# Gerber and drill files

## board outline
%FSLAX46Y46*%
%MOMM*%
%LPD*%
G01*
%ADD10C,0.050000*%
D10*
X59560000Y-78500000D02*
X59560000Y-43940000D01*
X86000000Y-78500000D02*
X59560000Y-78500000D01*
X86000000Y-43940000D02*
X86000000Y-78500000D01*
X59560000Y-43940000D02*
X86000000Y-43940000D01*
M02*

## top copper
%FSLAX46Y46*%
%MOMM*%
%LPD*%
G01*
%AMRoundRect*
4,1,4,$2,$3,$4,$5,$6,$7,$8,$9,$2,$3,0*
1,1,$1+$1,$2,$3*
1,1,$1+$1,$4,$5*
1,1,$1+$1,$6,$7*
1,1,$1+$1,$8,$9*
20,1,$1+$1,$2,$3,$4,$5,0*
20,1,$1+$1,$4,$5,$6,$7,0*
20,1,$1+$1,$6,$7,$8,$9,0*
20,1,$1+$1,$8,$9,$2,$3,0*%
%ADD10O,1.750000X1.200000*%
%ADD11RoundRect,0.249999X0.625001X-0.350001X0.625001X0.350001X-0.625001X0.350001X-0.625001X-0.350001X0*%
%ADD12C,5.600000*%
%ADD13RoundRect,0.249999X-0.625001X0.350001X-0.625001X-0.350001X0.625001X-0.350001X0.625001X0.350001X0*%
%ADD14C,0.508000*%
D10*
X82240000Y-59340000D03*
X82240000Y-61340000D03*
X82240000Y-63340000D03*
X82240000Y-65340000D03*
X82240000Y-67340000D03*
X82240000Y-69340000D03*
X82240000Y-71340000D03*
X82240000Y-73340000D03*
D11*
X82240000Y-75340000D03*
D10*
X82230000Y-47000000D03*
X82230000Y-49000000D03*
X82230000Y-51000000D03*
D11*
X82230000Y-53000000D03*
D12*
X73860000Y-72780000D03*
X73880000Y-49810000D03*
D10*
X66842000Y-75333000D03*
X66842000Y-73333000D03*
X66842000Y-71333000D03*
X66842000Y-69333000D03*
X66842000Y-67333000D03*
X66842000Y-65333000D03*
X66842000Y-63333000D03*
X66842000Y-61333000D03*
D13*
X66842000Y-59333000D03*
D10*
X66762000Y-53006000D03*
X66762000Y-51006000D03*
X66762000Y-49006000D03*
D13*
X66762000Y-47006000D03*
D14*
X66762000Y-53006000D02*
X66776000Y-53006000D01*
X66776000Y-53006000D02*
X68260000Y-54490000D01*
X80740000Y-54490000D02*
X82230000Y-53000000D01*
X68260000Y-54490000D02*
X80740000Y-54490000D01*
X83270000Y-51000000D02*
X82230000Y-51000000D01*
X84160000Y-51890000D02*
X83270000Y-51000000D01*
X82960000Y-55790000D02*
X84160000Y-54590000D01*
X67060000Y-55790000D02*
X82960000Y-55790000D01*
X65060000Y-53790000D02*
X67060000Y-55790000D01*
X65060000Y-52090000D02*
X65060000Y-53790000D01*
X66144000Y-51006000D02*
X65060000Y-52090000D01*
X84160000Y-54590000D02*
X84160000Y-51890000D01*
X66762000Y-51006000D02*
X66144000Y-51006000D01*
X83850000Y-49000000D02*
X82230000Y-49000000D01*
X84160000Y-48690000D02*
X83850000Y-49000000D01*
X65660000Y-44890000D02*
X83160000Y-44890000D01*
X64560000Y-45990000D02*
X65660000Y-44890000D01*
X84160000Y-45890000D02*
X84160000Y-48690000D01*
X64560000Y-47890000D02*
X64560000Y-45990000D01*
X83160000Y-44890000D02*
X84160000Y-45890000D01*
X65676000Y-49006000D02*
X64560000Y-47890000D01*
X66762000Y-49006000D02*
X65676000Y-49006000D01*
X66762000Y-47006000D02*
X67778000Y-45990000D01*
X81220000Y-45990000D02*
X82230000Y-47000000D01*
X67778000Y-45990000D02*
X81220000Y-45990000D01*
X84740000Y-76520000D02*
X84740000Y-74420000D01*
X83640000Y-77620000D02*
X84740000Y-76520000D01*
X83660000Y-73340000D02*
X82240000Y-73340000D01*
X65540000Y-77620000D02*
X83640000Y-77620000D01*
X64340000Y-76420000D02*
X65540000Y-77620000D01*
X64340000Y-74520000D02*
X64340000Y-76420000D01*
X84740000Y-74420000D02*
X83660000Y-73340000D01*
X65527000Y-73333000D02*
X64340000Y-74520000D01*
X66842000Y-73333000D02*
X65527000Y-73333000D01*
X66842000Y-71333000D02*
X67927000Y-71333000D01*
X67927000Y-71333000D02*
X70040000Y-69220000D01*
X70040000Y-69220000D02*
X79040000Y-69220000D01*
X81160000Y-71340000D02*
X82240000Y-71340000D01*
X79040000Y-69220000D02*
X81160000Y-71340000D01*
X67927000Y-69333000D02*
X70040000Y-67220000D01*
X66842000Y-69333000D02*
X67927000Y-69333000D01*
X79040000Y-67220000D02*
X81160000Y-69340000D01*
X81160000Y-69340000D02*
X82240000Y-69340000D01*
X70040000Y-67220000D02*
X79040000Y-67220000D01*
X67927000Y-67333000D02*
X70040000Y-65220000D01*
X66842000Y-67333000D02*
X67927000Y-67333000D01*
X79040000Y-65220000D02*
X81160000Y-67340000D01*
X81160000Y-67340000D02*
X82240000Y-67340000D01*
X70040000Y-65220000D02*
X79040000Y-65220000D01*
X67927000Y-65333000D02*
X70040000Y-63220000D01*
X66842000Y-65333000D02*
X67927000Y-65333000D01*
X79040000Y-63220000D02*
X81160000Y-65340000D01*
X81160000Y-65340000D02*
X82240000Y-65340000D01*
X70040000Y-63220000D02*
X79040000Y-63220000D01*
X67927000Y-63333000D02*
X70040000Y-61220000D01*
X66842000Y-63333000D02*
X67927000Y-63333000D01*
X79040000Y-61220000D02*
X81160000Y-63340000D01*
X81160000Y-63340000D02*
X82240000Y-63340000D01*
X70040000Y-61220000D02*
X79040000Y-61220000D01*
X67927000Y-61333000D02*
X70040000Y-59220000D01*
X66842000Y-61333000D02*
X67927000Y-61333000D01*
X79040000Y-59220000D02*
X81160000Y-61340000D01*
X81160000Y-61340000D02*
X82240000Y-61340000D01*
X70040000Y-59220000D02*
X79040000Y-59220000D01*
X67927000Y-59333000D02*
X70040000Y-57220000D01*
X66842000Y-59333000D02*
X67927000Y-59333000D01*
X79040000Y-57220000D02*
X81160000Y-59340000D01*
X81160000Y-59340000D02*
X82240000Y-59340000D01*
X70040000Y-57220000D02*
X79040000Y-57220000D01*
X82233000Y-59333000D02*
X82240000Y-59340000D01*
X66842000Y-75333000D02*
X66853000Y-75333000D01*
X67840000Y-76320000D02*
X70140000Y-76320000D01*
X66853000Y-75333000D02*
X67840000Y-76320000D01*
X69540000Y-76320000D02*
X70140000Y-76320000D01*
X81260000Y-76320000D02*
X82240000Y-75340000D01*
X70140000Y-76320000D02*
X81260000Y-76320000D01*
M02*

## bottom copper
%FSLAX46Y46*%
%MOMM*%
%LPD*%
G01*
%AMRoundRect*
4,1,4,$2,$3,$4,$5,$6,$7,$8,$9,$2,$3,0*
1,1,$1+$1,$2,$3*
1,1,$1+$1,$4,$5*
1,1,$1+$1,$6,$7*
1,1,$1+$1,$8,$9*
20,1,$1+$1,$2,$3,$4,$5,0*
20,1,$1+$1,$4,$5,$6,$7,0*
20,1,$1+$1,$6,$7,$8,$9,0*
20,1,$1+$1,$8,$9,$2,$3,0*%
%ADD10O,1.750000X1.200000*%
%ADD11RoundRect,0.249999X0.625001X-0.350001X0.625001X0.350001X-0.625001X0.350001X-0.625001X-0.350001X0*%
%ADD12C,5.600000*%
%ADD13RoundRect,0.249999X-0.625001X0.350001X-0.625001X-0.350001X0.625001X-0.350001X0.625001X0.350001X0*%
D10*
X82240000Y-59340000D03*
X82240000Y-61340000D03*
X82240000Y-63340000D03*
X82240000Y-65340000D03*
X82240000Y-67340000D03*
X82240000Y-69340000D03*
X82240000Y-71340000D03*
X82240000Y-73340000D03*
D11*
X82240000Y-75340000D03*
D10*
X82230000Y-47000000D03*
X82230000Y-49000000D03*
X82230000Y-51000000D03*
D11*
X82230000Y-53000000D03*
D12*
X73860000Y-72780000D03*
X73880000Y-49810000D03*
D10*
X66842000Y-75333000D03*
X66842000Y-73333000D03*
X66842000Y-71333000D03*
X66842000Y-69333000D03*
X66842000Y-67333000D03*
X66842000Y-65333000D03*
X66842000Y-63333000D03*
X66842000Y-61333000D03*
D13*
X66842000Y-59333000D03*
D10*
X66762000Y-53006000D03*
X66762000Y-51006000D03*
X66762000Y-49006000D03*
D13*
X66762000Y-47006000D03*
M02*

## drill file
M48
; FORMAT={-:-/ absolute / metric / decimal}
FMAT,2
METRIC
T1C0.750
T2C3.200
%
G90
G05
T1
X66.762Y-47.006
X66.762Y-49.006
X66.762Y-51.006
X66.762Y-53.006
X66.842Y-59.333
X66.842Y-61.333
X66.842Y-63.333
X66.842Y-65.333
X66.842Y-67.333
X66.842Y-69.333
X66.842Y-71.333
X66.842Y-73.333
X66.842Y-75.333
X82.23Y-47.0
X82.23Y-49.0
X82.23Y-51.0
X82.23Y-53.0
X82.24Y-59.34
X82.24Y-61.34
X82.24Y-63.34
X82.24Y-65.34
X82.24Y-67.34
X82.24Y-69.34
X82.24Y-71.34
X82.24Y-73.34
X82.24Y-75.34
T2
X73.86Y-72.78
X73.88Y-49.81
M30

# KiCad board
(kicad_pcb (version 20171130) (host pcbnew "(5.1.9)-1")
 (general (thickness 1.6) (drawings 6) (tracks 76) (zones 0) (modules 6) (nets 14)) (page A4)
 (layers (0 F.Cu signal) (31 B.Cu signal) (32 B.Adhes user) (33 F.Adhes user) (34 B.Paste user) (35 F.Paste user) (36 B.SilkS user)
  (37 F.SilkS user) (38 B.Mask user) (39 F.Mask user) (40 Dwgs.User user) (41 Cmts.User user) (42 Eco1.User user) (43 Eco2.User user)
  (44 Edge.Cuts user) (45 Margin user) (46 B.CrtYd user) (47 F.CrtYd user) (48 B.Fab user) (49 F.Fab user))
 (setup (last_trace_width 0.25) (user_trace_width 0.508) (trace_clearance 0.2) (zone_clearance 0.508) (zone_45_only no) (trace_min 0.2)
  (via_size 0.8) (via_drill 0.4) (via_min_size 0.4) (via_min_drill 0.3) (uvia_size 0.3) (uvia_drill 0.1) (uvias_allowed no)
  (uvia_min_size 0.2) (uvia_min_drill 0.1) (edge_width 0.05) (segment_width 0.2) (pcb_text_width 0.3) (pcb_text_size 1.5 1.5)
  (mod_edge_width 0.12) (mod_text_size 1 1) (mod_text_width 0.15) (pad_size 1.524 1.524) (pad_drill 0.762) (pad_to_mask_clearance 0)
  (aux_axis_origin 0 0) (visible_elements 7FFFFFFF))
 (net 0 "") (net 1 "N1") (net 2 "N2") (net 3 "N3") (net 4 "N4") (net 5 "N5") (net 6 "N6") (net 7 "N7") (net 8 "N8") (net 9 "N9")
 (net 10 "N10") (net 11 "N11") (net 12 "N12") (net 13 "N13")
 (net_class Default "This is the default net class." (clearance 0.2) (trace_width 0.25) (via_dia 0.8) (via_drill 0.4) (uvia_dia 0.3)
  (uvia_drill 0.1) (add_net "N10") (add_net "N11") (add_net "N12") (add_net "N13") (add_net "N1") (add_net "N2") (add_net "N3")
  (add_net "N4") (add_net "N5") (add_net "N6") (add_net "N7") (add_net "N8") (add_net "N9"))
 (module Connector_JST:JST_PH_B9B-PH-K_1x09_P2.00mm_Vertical (layer F.Cu) (at 82.24 75.34 90)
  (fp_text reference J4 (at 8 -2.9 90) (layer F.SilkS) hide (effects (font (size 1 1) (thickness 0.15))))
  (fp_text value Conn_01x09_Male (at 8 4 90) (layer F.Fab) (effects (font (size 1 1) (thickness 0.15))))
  (pad 9 thru_hole oval (at 16 0 90) (size 1.2 1.75) (drill 0.75) (layers *.Cu *.Mask) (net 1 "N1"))
  (pad 8 thru_hole oval (at 14 0 90) (size 1.2 1.75) (drill 0.75) (layers *.Cu *.Mask) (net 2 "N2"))
  (pad 7 thru_hole oval (at 12 0 90) (size 1.2 1.75) (drill 0.75) (layers *.Cu *.Mask) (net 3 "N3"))
  (pad 6 thru_hole oval (at 10 0 90) (size 1.2 1.75) (drill 0.75) (layers *.Cu *.Mask) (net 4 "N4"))
  (pad 5 thru_hole oval (at 8 0 90) (size 1.2 1.75) (drill 0.75) (layers *.Cu *.Mask) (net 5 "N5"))
  (pad 4 thru_hole oval (at 6 0 90) (size 1.2 1.75) (drill 0.75) (layers *.Cu *.Mask) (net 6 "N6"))
  (pad 3 thru_hole oval (at 4 0 90) (size 1.2 1.75) (drill 0.75) (layers *.Cu *.Mask) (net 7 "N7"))
  (pad 2 thru_hole oval (at 2 0 90) (size 1.2 1.75) (drill 0.75) (layers *.Cu *.Mask) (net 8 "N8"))
  (pad 1 thru_hole roundrect (at 0 0 90) (size 1.2 1.75) (drill 0.75) (layers *.Cu *.Mask) (roundrect_rratio 0.2083325) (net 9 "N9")))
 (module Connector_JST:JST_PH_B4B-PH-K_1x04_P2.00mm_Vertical (layer F.Cu) (at 82.23 53 90)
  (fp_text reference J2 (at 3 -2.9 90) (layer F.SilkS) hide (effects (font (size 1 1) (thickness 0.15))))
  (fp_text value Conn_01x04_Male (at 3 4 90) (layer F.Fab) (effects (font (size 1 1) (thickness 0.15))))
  (pad 4 thru_hole oval (at 6 0 90) (size 1.2 1.75) (drill 0.75) (layers *.Cu *.Mask) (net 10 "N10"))
  (pad 3 thru_hole oval (at 4 0 90) (size 1.2 1.75) (drill 0.75) (layers *.Cu *.Mask) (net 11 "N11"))
  (pad 2 thru_hole oval (at 2 0 90) (size 1.2 1.75) (drill 0.75) (layers *.Cu *.Mask) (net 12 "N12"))
  (pad 1 thru_hole roundrect (at 0 0 90) (size 1.2 1.75) (drill 0.75) (layers *.Cu *.Mask) (roundrect_rratio 0.2083325) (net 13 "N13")))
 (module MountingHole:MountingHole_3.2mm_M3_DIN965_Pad (layer F.Cu) (at 73.86 72.78)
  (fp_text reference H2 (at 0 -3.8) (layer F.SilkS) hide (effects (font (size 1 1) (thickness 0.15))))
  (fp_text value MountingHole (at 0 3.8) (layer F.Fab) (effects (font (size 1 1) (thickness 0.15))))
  (pad 1 thru_hole circle (at 0 0) (size 5.6 5.6) (drill 3.2) (layers *.Cu *.Mask)))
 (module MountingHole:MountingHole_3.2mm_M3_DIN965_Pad (layer F.Cu) (at 73.88 49.81)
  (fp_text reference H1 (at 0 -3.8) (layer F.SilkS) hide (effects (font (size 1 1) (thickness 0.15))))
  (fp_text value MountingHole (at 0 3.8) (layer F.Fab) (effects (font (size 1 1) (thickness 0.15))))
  (pad 1 thru_hole circle (at 0 0) (size 5.6 5.6) (drill 3.2) (layers *.Cu *.Mask)))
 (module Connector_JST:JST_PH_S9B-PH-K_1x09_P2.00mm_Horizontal (layer F.Cu) (at 66.842 59.333 270)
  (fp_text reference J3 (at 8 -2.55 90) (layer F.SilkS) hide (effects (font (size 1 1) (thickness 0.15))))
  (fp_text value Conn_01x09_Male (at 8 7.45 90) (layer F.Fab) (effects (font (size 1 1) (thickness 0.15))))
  (pad 9 thru_hole oval (at 16 0 270) (size 1.2 1.75) (drill 0.75) (layers *.Cu *.Mask) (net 9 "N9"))
  (pad 8 thru_hole oval (at 14 0 270) (size 1.2 1.75) (drill 0.75) (layers *.Cu *.Mask) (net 8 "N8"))
  (pad 7 thru_hole oval (at 12 0 270) (size 1.2 1.75) (drill 0.75) (layers *.Cu *.Mask) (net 7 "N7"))
  (pad 6 thru_hole oval (at 10 0 270) (size 1.2 1.75) (drill 0.75) (layers *.Cu *.Mask) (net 6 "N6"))
  (pad 5 thru_hole oval (at 8 0 270) (size 1.2 1.75) (drill 0.75) (layers *.Cu *.Mask) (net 5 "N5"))
  (pad 4 thru_hole oval (at 6 0 270) (size 1.2 1.75) (drill 0.75) (layers *.Cu *.Mask) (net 4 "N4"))
  (pad 3 thru_hole oval (at 4 0 270) (size 1.2 1.75) (drill 0.75) (layers *.Cu *.Mask) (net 3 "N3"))
  (pad 2 thru_hole oval (at 2 0 270) (size 1.2 1.75) (drill 0.75) (layers *.Cu *.Mask) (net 2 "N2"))
  (pad 1 thru_hole roundrect (at 0 0 270) (size 1.2 1.75) (drill 0.75) (layers *.Cu *.Mask) (roundrect_rratio 0.2083325) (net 1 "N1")))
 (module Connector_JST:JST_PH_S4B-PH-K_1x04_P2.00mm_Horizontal (layer F.Cu) (at 66.762 47.006 270)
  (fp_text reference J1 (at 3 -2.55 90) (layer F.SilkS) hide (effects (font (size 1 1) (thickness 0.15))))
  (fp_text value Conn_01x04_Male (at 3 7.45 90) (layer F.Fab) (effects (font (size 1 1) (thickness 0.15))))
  (pad 4 thru_hole oval (at 6 0 270) (size 1.2 1.75) (drill 0.75) (layers *.Cu *.Mask) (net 13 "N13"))
  (pad 3 thru_hole oval (at 4 0 270) (size 1.2 1.75) (drill 0.75) (layers *.Cu *.Mask) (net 12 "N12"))
  (pad 2 thru_hole oval (at 2 0 270) (size 1.2 1.75) (drill 0.75) (layers *.Cu *.Mask) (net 11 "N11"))
  (pad 1 thru_hole roundrect (at 0 0 270) (size 1.2 1.75) (drill 0.75) (layers *.Cu *.Mask) (roundrect_rratio 0.2083325) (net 10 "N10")))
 (gr_line (start 59.56 78.5) (end 59.56 43.94) (layer Edge.Cuts) (width 0.05))
 (gr_line (start 86 78.5) (end 59.56 78.5) (layer Edge.Cuts) (width 0.05))
 (gr_line (start 86 43.94) (end 86 78.5) (layer Edge.Cuts) (width 0.05))
 (gr_line (start 59.56 43.94) (end 86 43.94) (layer Edge.Cuts) (width 0.05))
 (segment (start 66.762 53.006) (end 66.776 53.006) (width 0.508) (layer F.Cu) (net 13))
 (segment (start 66.776 53.006) (end 68.26 54.49) (width 0.508) (layer F.Cu) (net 13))
 (segment (start 80.74 54.49) (end 82.23 53) (width 0.508) (layer F.Cu) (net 13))
 (segment (start 68.26 54.49) (end 80.74 54.49) (width 0.508) (layer F.Cu) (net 13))
 (segment (start 83.27 51) (end 82.23 51) (width 0.508) (layer F.Cu) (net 12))
 (segment (start 84.16 51.89) (end 83.27 51) (width 0.508) (layer F.Cu) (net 12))
 (segment (start 82.96 55.79) (end 84.16 54.59) (width 0.508) (layer F.Cu) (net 12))
 (segment (start 67.06 55.79) (end 82.96 55.79) (width 0.508) (layer F.Cu) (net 12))
 (segment (start 65.06 53.79) (end 67.06 55.79) (width 0.508) (layer F.Cu) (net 12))
 (segment (start 65.06 52.09) (end 65.06 53.79) (width 0.508) (layer F.Cu) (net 12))
 (segment (start 66.144 51.006) (end 65.06 52.09) (width 0.508) (layer F.Cu) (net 12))
 (segment (start 84.16 54.59) (end 84.16 51.89) (width 0.508) (layer F.Cu) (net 12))
 (segment (start 66.762 51.006) (end 66.144 51.006) (width 0.508) (layer F.Cu) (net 12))
 (segment (start 83.85 49) (end 82.23 49) (width 0.508) (layer F.Cu) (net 11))
 (segment (start 84.16 48.69) (end 83.85 49) (width 0.508) (layer F.Cu) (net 11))
 (segment (start 65.66 44.89) (end 83.16 44.89) (width 0.508) (layer F.Cu) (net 11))
 (segment (start 64.56 45.99) (end 65.66 44.89) (width 0.508) (layer F.Cu) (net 11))
 (segment (start 84.16 45.89) (end 84.16 48.69) (width 0.508) (layer F.Cu) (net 11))
 (segment (start 64.56 47.89) (end 64.56 45.99) (width 0.508) (layer F.Cu) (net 11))
 (segment (start 83.16 44.89) (end 84.16 45.89) (width 0.508) (layer F.Cu) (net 11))
 (segment (start 65.676 49.006) (end 64.56 47.89) (width 0.508) (layer F.Cu) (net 11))
 (segment (start 66.762 49.006) (end 65.676 49.006) (width 0.508) (layer F.Cu) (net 11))
 (segment (start 66.762 47.006) (end 67.778 45.99) (width 0.508) (layer F.Cu) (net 10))
 (segment (start 81.22 45.99) (end 82.23 47) (width 0.508) (layer F.Cu) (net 10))
 (segment (start 67.778 45.99) (end 81.22 45.99) (width 0.508) (layer F.Cu) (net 10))
 (segment (start 84.74 76.52) (end 84.74 74.42) (width 0.508) (layer F.Cu) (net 8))
 (segment (start 83.64 77.62) (end 84.74 76.52) (width 0.508) (layer F.Cu) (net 8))
 (segment (start 83.66 73.34) (end 82.24 73.34) (width 0.508) (layer F.Cu) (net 8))
 (segment (start 65.54 77.62) (end 83.64 77.62) (width 0.508) (layer F.Cu) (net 8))
 (segment (start 64.34 76.42) (end 65.54 77.62) (width 0.508) (layer F.Cu) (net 8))
 (segment (start 64.34 74.52) (end 64.34 76.42) (width 0.508) (layer F.Cu) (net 8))
 (segment (start 84.74 74.42) (end 83.66 73.34) (width 0.508) (layer F.Cu) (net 8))
 (segment (start 65.527 73.333) (end 64.34 74.52) (width 0.508) (layer F.Cu) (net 8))
 (segment (start 66.842 73.333) (end 65.527 73.333) (width 0.508) (layer F.Cu) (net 8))
 (segment (start 66.842 71.333) (end 67.927 71.333) (width 0.508) (layer F.Cu) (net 7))
 (segment (start 67.927 71.333) (end 70.04 69.22) (width 0.508) (layer F.Cu) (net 7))
 (segment (start 70.04 69.22) (end 79.04 69.22) (width 0.508) (layer F.Cu) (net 7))
 (segment (start 81.16 71.34) (end 82.24 71.34) (width 0.508) (layer F.Cu) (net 7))
 (segment (start 79.04 69.22) (end 81.16 71.34) (width 0.508) (layer F.Cu) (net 7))
 (segment (start 67.927 69.333) (end 70.04 67.22) (width 0.508) (layer F.Cu) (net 6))
 (segment (start 66.842 69.333) (end 67.927 69.333) (width 0.508) (layer F.Cu) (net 6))
 (segment (start 79.04 67.22) (end 81.16 69.34) (width 0.508) (layer F.Cu) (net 6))
 (segment (start 81.16 69.34) (end 82.24 69.34) (width 0.508) (layer F.Cu) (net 6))
 (segment (start 70.04 67.22) (end 79.04 67.22) (width 0.508) (layer F.Cu) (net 6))
 (segment (start 67.927 67.333) (end 70.04 65.22) (width 0.508) (layer F.Cu) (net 5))
 (segment (start 66.842 67.333) (end 67.927 67.333) (width 0.508) (layer F.Cu) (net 5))
 (segment (start 79.04 65.22) (end 81.16 67.34) (width 0.508) (layer F.Cu) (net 5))
 (segment (start 81.16 67.34) (end 82.24 67.34) (width 0.508) (layer F.Cu) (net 5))
 (segment (start 70.04 65.22) (end 79.04 65.22) (width 0.508) (layer F.Cu) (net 5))
 (segment (start 67.927 65.333) (end 70.04 63.22) (width 0.508) (layer F.Cu) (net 4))
 (segment (start 66.842 65.333) (end 67.927 65.333) (width 0.508) (layer F.Cu) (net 4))
 (segment (start 79.04 63.22) (end 81.16 65.34) (width 0.508) (layer F.Cu) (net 4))
 (segment (start 81.16 65.34) (end 82.24 65.34) (width 0.508) (layer F.Cu) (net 4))
 (segment (start 70.04 63.22) (end 79.04 63.22) (width 0.508) (layer F.Cu) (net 4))
 (segment (start 67.927 63.333) (end 70.04 61.22) (width 0.508) (layer F.Cu) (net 3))
 (segment (start 66.842 63.333) (end 67.927 63.333) (width 0.508) (layer F.Cu) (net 3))
 (segment (start 79.04 61.22) (end 81.16 63.34) (width 0.508) (layer F.Cu) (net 3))
 (segment (start 81.16 63.34) (end 82.24 63.34) (width 0.508) (layer F.Cu) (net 3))
 (segment (start 70.04 61.22) (end 79.04 61.22) (width 0.508) (layer F.Cu) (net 3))
 (segment (start 67.927 61.333) (end 70.04 59.22) (width 0.508) (layer F.Cu) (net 2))
 (segment (start 66.842 61.333) (end 67.927 61.333) (width 0.508) (layer F.Cu) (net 2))
 (segment (start 79.04 59.22) (end 81.16 61.34) (width 0.508) (layer F.Cu) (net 2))
 (segment (start 81.16 61.34) (end 82.24 61.34) (width 0.508) (layer F.Cu) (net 2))
 (segment (start 70.04 59.22) (end 79.04 59.22) (width 0.508) (layer F.Cu) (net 2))
 (segment (start 67.927 59.333) (end 70.04 57.22) (width 0.508) (layer F.Cu) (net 1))
 (segment (start 66.842 59.333) (end 67.927 59.333) (width 0.508) (layer F.Cu) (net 1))
 (segment (start 79.04 57.22) (end 81.16 59.34) (width 0.508) (layer F.Cu) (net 1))
 (segment (start 81.16 59.34) (end 82.24 59.34) (width 0.508) (layer F.Cu) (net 1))
 (segment (start 70.04 57.22) (end 79.04 57.22) (width 0.508) (layer F.Cu) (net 1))
 (segment (start 82.233 59.333) (end 82.24 59.34) (width 0.508) (layer F.Cu) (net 1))
 (segment (start 66.842 75.333) (end 66.853 75.333) (width 0.508) (layer F.Cu) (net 9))
 (segment (start 67.84 76.32) (end 70.14 76.32) (width 0.508) (layer F.Cu) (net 9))
 (segment (start 66.853 75.333) (end 67.84 76.32) (width 0.508) (layer F.Cu) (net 9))
 (segment (start 69.54 76.32) (end 70.14 76.32) (width 0.508) (layer F.Cu) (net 9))
 (segment (start 81.26 76.32) (end 82.24 75.34) (width 0.508) (layer F.Cu) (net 9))
 (segment (start 70.14 76.32) (end 81.26 76.32) (width 0.508) (layer F.Cu) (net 9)))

